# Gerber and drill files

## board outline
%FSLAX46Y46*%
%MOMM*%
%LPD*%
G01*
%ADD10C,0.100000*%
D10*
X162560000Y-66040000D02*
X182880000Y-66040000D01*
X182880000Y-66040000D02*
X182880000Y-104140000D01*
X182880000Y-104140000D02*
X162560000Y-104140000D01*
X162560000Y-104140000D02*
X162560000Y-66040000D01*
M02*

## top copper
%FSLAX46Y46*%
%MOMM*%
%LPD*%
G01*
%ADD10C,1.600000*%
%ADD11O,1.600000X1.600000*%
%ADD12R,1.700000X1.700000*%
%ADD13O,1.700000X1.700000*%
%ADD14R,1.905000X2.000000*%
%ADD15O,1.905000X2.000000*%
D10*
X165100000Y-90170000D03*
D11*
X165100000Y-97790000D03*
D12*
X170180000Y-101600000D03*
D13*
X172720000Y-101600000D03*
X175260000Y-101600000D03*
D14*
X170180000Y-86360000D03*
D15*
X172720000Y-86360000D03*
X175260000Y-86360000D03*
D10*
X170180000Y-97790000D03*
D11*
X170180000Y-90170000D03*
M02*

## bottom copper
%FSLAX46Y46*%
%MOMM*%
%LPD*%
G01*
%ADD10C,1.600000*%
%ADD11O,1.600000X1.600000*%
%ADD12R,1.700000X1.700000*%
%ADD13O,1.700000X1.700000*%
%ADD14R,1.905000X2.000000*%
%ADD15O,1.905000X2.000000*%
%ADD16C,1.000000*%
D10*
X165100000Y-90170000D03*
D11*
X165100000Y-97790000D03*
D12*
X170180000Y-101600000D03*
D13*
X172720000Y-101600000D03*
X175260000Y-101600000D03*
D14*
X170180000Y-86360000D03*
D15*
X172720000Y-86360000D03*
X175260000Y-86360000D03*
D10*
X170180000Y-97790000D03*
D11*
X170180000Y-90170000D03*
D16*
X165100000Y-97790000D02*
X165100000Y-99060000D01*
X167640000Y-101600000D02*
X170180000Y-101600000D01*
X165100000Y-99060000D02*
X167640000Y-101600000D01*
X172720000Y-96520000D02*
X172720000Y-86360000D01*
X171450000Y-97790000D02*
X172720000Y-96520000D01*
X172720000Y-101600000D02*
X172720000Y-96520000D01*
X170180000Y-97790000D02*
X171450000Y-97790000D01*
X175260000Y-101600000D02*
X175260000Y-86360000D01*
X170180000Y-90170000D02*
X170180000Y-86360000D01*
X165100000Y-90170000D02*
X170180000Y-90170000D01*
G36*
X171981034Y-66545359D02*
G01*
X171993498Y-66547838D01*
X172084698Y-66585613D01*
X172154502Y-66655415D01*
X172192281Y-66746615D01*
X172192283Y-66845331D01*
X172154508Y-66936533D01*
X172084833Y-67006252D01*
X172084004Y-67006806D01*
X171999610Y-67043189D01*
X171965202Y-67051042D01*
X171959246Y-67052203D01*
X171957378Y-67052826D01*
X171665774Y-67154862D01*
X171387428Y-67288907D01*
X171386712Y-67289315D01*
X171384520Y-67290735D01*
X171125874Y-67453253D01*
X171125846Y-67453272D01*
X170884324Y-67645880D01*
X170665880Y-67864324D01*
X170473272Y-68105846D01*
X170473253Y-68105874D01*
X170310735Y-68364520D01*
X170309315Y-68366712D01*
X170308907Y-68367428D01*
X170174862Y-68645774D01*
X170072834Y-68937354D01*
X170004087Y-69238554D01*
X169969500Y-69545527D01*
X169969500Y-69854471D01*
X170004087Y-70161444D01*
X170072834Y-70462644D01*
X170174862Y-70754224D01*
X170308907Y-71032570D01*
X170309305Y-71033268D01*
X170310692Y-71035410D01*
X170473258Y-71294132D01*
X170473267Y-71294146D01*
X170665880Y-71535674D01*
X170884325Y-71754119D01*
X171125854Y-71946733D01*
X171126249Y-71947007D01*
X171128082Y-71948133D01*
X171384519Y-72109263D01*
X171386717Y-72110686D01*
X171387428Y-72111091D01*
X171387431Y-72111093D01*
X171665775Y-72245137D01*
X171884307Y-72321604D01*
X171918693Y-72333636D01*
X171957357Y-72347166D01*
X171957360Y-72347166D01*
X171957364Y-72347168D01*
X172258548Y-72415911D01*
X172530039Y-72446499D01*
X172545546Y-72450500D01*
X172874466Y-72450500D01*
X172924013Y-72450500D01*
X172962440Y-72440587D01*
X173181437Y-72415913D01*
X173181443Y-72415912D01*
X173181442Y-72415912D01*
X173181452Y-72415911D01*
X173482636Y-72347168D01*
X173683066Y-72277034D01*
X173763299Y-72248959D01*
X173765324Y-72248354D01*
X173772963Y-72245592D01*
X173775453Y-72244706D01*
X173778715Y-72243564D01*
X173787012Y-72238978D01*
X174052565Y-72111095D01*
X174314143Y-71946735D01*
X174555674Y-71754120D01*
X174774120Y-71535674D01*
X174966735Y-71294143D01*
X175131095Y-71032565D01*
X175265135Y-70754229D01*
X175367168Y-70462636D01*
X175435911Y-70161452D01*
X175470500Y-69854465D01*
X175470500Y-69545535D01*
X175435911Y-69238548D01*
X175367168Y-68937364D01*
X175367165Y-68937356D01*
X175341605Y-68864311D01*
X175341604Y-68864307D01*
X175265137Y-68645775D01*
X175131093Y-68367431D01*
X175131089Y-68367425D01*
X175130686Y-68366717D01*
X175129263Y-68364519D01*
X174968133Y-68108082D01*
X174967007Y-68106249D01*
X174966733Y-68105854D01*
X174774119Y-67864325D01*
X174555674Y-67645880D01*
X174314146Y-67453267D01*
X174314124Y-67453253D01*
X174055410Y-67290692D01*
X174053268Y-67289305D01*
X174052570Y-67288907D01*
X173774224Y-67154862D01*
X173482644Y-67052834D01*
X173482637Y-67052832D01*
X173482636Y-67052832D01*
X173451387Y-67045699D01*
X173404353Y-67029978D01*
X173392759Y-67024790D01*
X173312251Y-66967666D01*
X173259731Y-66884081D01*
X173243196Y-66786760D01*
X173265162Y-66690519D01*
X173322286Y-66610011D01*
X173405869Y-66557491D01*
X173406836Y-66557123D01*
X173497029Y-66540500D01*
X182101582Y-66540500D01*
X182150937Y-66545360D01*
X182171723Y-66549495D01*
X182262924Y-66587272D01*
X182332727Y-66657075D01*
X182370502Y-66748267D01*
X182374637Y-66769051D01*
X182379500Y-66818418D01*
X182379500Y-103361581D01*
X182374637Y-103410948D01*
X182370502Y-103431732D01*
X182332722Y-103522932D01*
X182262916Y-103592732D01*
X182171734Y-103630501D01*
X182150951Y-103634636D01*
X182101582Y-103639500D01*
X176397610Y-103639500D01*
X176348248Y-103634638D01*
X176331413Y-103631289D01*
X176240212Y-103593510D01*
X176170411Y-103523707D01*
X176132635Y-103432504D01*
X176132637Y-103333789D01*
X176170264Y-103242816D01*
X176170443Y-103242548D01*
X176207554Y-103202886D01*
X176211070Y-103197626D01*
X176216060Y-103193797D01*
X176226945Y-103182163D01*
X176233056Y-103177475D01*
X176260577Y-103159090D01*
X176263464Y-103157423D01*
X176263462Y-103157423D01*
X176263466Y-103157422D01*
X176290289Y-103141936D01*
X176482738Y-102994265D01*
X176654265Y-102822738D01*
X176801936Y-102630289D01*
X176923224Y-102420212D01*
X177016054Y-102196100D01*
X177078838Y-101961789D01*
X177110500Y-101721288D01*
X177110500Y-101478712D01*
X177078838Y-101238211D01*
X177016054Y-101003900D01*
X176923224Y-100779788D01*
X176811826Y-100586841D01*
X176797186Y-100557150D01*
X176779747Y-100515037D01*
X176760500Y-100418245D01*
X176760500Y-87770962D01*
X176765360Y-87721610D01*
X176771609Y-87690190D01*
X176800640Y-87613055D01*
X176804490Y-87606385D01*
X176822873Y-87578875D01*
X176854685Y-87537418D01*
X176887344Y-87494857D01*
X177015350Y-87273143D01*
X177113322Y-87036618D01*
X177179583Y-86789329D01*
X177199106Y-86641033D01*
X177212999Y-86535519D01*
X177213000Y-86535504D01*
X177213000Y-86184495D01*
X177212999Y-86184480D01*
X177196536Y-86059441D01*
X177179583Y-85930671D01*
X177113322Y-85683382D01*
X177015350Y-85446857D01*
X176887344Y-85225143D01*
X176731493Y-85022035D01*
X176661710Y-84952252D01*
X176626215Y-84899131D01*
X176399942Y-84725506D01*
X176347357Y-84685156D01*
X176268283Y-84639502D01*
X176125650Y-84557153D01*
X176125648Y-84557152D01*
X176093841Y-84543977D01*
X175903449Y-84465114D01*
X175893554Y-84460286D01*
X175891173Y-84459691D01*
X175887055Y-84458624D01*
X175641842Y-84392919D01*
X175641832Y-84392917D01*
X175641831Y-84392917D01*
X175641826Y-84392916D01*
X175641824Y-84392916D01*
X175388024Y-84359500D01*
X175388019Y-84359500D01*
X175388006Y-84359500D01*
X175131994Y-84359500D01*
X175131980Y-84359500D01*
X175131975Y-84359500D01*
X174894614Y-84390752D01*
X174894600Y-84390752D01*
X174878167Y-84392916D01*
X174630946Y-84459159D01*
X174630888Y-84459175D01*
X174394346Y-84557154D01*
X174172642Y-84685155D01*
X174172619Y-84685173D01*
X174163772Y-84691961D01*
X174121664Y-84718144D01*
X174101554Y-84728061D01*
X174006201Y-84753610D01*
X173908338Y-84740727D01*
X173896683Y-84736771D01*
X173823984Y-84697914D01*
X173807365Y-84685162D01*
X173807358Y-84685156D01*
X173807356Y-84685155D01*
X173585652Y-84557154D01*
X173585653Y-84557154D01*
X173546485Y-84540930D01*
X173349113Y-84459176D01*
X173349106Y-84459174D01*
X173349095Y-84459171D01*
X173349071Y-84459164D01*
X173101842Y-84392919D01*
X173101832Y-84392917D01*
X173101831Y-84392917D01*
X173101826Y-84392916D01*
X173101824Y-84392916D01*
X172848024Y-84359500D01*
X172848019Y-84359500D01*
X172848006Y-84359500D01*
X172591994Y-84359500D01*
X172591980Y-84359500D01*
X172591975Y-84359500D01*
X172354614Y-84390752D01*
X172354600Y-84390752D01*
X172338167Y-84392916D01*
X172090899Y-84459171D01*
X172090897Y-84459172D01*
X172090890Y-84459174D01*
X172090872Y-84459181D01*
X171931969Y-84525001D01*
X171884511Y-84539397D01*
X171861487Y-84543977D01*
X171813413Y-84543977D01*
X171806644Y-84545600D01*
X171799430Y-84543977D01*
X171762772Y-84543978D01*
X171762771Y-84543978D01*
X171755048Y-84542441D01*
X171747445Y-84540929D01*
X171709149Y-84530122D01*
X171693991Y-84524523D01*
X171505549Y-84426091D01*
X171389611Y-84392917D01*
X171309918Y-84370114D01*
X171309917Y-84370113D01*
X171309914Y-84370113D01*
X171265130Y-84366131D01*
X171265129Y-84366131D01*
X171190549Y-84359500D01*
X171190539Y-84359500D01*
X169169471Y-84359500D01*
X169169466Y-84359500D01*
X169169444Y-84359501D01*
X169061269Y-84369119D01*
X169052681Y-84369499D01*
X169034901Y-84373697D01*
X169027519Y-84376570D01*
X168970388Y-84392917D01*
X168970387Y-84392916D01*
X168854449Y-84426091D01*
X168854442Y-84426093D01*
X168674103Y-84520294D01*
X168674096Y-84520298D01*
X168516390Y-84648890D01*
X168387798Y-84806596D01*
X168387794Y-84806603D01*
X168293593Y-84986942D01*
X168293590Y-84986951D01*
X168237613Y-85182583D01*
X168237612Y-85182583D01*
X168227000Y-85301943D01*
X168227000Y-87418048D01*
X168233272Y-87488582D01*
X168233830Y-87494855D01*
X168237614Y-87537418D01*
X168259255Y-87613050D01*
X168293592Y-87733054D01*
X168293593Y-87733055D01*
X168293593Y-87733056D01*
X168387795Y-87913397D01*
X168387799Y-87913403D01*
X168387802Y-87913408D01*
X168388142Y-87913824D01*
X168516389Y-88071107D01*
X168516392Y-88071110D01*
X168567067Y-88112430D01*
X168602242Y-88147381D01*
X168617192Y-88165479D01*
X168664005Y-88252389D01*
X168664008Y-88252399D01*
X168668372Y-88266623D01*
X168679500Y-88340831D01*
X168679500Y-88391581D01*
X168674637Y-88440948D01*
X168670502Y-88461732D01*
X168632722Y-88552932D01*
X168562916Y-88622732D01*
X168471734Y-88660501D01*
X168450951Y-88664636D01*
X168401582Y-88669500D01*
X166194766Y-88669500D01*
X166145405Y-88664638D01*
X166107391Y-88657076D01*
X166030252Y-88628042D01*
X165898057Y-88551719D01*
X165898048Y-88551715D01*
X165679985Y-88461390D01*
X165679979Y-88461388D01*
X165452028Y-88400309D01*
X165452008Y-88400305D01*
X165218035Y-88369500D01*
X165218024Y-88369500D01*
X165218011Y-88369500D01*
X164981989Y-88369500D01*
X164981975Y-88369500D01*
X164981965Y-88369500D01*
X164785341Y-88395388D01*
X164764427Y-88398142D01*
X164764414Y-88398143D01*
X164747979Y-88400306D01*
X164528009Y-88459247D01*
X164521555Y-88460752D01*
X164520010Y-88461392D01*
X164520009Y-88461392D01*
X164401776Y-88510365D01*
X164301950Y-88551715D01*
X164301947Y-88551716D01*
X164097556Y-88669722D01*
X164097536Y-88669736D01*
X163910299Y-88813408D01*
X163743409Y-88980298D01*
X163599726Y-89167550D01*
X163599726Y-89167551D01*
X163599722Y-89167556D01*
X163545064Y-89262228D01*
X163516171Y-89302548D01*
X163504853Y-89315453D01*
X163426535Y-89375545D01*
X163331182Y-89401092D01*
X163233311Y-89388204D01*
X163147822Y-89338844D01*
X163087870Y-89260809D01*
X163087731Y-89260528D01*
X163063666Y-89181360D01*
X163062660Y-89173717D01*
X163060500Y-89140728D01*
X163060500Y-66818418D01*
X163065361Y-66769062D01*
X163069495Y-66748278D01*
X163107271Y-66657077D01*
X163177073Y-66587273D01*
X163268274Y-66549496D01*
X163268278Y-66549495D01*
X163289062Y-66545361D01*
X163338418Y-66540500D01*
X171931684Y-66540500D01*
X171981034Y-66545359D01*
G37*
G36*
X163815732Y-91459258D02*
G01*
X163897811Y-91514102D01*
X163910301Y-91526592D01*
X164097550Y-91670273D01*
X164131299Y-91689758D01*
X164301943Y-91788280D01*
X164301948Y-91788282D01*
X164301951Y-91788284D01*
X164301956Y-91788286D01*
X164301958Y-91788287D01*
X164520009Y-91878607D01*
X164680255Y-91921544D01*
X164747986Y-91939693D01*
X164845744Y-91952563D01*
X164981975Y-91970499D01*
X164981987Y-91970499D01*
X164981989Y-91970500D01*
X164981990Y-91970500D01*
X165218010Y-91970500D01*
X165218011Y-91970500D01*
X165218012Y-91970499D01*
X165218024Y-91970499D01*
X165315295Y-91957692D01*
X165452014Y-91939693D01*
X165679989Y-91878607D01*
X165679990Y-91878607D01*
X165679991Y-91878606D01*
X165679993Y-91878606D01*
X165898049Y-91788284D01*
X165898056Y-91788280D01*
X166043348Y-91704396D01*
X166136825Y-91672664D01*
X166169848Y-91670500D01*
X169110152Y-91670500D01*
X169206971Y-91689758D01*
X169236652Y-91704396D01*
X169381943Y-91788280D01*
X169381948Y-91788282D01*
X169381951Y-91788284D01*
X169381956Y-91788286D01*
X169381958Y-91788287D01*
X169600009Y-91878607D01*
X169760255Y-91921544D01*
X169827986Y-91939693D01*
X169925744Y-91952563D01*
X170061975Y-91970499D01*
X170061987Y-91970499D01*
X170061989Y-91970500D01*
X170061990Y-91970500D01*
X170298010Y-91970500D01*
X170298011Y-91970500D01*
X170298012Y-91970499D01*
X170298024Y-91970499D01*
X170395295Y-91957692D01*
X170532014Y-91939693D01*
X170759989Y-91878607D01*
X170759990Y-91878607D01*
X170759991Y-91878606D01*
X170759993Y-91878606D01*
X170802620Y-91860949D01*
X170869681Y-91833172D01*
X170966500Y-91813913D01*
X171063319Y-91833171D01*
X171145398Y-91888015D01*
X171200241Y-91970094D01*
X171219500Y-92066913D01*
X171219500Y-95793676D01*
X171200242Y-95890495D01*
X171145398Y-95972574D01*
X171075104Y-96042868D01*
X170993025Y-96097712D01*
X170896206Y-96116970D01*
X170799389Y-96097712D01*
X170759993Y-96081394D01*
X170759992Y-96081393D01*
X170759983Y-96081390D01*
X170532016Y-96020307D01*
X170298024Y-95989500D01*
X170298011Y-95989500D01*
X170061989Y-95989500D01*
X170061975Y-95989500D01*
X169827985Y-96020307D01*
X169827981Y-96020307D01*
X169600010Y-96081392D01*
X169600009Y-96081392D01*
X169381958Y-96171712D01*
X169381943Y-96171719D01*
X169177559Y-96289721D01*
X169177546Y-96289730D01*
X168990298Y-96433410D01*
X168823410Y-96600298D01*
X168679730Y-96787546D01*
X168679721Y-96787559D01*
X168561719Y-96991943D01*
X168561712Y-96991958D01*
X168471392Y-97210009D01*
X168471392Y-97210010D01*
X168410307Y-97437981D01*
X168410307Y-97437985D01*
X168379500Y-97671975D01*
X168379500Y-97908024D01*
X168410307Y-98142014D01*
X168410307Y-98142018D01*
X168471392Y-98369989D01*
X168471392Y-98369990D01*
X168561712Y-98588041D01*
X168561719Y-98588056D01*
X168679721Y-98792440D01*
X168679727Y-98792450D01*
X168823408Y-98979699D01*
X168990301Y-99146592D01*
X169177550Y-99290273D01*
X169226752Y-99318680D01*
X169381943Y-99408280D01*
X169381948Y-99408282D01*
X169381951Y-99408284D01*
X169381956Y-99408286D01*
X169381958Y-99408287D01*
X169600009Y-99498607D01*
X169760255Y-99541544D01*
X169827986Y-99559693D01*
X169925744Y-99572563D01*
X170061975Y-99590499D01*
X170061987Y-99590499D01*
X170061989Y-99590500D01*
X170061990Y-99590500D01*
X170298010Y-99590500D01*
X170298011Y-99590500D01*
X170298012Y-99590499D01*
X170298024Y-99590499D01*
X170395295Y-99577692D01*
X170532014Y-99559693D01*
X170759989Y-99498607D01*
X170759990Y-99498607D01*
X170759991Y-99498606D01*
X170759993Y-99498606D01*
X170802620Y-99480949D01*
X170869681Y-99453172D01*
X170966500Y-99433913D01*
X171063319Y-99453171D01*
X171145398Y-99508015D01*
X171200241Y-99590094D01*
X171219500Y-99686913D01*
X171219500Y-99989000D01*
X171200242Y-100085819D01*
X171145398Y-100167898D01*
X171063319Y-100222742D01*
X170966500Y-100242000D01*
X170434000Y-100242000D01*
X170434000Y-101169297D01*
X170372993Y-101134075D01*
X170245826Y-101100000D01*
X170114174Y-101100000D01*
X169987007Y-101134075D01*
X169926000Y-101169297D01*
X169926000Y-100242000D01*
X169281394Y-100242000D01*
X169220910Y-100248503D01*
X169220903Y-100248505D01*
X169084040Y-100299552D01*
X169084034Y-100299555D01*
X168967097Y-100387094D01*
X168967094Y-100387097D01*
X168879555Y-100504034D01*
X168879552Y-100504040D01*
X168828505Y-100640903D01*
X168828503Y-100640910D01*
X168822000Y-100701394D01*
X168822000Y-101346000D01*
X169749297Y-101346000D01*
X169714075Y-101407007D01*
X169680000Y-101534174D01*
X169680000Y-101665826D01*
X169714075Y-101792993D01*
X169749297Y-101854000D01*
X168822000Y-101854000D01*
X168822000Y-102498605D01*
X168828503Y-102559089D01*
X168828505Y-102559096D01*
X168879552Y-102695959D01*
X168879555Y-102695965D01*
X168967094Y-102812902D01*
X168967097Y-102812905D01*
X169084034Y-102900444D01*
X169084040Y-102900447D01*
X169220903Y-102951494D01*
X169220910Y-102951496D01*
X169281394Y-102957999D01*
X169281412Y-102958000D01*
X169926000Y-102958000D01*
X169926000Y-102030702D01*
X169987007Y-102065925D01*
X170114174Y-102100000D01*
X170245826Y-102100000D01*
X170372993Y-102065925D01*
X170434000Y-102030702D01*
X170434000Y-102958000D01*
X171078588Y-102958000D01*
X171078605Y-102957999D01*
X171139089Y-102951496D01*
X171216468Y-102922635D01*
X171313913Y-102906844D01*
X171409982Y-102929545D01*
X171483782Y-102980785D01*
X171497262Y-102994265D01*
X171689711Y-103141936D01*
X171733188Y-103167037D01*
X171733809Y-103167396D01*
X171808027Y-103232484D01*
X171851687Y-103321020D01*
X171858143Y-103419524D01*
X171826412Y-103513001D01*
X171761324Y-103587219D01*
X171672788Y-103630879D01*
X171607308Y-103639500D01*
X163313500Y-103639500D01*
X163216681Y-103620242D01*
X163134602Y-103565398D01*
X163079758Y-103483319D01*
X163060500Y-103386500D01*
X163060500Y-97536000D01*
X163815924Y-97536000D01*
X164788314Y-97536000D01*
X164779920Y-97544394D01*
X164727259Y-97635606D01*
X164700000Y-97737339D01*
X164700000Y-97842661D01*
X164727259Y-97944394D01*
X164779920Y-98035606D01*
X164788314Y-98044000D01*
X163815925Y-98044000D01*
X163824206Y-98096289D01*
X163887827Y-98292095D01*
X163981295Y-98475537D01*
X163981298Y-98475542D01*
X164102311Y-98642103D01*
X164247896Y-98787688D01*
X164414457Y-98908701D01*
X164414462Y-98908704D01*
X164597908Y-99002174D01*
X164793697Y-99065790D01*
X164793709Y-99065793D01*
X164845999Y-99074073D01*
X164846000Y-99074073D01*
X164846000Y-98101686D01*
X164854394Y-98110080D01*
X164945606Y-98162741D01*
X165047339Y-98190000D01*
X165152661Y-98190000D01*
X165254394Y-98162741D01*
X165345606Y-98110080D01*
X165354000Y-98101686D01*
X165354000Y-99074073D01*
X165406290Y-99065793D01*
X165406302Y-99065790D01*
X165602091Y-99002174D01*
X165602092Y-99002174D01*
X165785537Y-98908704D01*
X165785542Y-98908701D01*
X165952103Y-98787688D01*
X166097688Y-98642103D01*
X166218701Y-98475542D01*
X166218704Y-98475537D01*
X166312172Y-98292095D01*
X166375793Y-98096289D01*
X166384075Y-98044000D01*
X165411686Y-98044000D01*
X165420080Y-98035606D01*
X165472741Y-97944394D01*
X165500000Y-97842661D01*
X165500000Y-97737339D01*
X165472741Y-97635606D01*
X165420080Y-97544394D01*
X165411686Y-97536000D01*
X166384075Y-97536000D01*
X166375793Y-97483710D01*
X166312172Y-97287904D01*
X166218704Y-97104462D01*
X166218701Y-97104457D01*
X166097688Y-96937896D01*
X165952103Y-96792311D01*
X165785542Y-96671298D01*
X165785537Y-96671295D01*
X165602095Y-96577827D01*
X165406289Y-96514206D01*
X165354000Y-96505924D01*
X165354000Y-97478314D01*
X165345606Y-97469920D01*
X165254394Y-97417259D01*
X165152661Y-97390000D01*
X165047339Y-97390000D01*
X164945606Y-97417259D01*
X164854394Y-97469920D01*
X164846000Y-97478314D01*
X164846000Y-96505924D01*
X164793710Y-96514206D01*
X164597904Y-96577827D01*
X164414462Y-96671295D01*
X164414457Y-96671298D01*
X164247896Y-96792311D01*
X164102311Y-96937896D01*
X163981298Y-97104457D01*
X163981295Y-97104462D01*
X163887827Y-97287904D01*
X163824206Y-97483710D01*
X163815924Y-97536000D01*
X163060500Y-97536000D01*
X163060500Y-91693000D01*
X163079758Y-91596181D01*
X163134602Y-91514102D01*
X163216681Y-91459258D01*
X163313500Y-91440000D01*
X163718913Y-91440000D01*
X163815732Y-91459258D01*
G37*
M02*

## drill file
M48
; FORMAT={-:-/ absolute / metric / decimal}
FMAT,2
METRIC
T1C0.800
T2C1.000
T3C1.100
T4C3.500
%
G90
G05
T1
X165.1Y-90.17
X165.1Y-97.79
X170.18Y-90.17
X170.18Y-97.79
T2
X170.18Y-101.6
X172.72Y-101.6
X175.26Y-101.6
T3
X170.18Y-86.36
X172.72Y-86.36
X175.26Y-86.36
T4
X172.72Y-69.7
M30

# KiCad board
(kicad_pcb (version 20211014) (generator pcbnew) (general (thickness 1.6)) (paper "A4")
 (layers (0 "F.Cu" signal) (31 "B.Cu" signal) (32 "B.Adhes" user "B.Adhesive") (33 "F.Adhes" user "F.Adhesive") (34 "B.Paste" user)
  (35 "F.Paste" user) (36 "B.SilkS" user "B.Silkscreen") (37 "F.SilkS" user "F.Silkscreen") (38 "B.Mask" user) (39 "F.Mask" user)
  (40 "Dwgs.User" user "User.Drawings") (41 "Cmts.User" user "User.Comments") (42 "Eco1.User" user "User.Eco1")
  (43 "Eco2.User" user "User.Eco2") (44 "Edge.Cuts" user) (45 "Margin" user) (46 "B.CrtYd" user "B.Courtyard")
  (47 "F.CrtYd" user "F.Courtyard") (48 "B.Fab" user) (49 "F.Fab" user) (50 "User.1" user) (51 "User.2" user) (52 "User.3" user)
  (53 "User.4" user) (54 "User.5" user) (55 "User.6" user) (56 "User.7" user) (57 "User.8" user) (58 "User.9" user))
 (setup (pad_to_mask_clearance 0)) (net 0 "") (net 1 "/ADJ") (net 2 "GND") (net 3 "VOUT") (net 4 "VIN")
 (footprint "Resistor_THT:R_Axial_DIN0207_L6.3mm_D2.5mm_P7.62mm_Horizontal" (layer "F.Cu") (at 165.1 90.17 -90)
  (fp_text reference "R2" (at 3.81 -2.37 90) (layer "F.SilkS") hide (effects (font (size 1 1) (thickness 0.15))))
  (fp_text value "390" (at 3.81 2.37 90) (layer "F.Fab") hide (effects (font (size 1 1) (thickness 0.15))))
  (pad "1" thru_hole circle (at 0 0 270) (size 1.6 1.6) (drill 0.8) (layers *.Cu *.Mask) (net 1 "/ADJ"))
  (pad "2" thru_hole oval (at 7.62 0 270) (size 1.6 1.6) (drill 0.8) (layers *.Cu *.Mask) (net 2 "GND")))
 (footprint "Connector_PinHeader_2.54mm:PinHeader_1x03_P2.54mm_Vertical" (layer "F.Cu") (at 170.18 101.6 90)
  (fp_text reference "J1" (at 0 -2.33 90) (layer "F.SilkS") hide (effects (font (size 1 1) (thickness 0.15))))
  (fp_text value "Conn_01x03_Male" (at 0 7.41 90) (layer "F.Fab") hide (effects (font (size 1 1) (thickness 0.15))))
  (pad "1" thru_hole rect (at 0 0 90) (size 1.7 1.7) (drill 1) (layers *.Cu *.Mask) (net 2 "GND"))
  (pad "2" thru_hole oval (at 0 2.54 90) (size 1.7 1.7) (drill 1) (layers *.Cu *.Mask) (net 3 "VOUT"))
  (pad "3" thru_hole oval (at 0 5.08 90) (size 1.7 1.7) (drill 1) (layers *.Cu *.Mask) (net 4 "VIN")))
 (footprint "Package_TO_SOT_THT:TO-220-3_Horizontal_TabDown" (layer "F.Cu") (at 170.18 86.36)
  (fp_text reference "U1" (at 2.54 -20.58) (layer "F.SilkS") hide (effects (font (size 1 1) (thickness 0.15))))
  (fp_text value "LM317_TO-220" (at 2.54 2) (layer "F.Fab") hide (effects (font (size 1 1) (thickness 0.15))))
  (pad "" np_thru_hole oval (at 2.54 -16.66) (size 3.5 3.5) (drill 3.5) (layers *.Cu *.Mask))
  (pad "1" thru_hole rect (at 0 0) (size 1.905 2) (drill 1.1) (layers *.Cu *.Mask) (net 1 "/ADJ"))
  (pad "2" thru_hole oval (at 2.54 0) (size 1.905 2) (drill 1.1) (layers *.Cu *.Mask) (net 3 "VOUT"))
  (pad "3" thru_hole oval (at 5.08 0) (size 1.905 2) (drill 1.1) (layers *.Cu *.Mask) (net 4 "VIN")))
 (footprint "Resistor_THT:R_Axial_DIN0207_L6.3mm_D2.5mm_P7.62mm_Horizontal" (layer "F.Cu") (at 170.18 97.79 90)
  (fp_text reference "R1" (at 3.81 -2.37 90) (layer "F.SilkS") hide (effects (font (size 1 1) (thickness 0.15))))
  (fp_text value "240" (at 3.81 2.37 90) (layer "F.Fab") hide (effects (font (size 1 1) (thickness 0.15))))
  (pad "1" thru_hole circle (at 0 0 90) (size 1.6 1.6) (drill 0.8) (layers *.Cu *.Mask) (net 3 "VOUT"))
  (pad "2" thru_hole oval (at 7.62 0 90) (size 1.6 1.6) (drill 0.8) (layers *.Cu *.Mask) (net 1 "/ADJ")))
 (gr_line (start 162.56 66.04) (end 182.88 66.04) (layer "Edge.Cuts") (width 0.1))
 (gr_line (start 182.88 66.04) (end 182.88 104.14) (layer "Edge.Cuts") (width 0.1))
 (gr_line (start 182.88 104.14) (end 162.56 104.14) (layer "Edge.Cuts") (width 0.1))
 (gr_line (start 162.56 104.14) (end 162.56 66.04) (layer "Edge.Cuts") (width 0.1))
 (segment (start 165.1 97.79) (end 165.1 99.06) (width 1) (layer "B.Cu") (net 2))
 (segment (start 167.64 101.6) (end 170.18 101.6) (width 1) (layer "B.Cu") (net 2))
 (segment (start 165.1 99.06) (end 167.64 101.6) (width 1) (layer "B.Cu") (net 2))
 (segment (start 172.72 96.52) (end 172.72 86.36) (width 1) (layer "B.Cu") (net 3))
 (segment (start 171.45 97.79) (end 172.72 96.52) (width 1) (layer "B.Cu") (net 3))
 (segment (start 172.72 101.6) (end 172.72 96.52) (width 1) (layer "B.Cu") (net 3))
 (segment (start 170.18 97.79) (end 171.45 97.79) (width 1) (layer "B.Cu") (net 3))
 (segment (start 175.26 101.6) (end 175.26 86.36) (width 1) (layer "B.Cu") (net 4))
 (segment (start 170.18 90.17) (end 170.18 86.36) (width 1) (layer "B.Cu") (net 1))
 (segment (start 165.1 90.17) (end 170.18 90.17) (width 1) (layer "B.Cu") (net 1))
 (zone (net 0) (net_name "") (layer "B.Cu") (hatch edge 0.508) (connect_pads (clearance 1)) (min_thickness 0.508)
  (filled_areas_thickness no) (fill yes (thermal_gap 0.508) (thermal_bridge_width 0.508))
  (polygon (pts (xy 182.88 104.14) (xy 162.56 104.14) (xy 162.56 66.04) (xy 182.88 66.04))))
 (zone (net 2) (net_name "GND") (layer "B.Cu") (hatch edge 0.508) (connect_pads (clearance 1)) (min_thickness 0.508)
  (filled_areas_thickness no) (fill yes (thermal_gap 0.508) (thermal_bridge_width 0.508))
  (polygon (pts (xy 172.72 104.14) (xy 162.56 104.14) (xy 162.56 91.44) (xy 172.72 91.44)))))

